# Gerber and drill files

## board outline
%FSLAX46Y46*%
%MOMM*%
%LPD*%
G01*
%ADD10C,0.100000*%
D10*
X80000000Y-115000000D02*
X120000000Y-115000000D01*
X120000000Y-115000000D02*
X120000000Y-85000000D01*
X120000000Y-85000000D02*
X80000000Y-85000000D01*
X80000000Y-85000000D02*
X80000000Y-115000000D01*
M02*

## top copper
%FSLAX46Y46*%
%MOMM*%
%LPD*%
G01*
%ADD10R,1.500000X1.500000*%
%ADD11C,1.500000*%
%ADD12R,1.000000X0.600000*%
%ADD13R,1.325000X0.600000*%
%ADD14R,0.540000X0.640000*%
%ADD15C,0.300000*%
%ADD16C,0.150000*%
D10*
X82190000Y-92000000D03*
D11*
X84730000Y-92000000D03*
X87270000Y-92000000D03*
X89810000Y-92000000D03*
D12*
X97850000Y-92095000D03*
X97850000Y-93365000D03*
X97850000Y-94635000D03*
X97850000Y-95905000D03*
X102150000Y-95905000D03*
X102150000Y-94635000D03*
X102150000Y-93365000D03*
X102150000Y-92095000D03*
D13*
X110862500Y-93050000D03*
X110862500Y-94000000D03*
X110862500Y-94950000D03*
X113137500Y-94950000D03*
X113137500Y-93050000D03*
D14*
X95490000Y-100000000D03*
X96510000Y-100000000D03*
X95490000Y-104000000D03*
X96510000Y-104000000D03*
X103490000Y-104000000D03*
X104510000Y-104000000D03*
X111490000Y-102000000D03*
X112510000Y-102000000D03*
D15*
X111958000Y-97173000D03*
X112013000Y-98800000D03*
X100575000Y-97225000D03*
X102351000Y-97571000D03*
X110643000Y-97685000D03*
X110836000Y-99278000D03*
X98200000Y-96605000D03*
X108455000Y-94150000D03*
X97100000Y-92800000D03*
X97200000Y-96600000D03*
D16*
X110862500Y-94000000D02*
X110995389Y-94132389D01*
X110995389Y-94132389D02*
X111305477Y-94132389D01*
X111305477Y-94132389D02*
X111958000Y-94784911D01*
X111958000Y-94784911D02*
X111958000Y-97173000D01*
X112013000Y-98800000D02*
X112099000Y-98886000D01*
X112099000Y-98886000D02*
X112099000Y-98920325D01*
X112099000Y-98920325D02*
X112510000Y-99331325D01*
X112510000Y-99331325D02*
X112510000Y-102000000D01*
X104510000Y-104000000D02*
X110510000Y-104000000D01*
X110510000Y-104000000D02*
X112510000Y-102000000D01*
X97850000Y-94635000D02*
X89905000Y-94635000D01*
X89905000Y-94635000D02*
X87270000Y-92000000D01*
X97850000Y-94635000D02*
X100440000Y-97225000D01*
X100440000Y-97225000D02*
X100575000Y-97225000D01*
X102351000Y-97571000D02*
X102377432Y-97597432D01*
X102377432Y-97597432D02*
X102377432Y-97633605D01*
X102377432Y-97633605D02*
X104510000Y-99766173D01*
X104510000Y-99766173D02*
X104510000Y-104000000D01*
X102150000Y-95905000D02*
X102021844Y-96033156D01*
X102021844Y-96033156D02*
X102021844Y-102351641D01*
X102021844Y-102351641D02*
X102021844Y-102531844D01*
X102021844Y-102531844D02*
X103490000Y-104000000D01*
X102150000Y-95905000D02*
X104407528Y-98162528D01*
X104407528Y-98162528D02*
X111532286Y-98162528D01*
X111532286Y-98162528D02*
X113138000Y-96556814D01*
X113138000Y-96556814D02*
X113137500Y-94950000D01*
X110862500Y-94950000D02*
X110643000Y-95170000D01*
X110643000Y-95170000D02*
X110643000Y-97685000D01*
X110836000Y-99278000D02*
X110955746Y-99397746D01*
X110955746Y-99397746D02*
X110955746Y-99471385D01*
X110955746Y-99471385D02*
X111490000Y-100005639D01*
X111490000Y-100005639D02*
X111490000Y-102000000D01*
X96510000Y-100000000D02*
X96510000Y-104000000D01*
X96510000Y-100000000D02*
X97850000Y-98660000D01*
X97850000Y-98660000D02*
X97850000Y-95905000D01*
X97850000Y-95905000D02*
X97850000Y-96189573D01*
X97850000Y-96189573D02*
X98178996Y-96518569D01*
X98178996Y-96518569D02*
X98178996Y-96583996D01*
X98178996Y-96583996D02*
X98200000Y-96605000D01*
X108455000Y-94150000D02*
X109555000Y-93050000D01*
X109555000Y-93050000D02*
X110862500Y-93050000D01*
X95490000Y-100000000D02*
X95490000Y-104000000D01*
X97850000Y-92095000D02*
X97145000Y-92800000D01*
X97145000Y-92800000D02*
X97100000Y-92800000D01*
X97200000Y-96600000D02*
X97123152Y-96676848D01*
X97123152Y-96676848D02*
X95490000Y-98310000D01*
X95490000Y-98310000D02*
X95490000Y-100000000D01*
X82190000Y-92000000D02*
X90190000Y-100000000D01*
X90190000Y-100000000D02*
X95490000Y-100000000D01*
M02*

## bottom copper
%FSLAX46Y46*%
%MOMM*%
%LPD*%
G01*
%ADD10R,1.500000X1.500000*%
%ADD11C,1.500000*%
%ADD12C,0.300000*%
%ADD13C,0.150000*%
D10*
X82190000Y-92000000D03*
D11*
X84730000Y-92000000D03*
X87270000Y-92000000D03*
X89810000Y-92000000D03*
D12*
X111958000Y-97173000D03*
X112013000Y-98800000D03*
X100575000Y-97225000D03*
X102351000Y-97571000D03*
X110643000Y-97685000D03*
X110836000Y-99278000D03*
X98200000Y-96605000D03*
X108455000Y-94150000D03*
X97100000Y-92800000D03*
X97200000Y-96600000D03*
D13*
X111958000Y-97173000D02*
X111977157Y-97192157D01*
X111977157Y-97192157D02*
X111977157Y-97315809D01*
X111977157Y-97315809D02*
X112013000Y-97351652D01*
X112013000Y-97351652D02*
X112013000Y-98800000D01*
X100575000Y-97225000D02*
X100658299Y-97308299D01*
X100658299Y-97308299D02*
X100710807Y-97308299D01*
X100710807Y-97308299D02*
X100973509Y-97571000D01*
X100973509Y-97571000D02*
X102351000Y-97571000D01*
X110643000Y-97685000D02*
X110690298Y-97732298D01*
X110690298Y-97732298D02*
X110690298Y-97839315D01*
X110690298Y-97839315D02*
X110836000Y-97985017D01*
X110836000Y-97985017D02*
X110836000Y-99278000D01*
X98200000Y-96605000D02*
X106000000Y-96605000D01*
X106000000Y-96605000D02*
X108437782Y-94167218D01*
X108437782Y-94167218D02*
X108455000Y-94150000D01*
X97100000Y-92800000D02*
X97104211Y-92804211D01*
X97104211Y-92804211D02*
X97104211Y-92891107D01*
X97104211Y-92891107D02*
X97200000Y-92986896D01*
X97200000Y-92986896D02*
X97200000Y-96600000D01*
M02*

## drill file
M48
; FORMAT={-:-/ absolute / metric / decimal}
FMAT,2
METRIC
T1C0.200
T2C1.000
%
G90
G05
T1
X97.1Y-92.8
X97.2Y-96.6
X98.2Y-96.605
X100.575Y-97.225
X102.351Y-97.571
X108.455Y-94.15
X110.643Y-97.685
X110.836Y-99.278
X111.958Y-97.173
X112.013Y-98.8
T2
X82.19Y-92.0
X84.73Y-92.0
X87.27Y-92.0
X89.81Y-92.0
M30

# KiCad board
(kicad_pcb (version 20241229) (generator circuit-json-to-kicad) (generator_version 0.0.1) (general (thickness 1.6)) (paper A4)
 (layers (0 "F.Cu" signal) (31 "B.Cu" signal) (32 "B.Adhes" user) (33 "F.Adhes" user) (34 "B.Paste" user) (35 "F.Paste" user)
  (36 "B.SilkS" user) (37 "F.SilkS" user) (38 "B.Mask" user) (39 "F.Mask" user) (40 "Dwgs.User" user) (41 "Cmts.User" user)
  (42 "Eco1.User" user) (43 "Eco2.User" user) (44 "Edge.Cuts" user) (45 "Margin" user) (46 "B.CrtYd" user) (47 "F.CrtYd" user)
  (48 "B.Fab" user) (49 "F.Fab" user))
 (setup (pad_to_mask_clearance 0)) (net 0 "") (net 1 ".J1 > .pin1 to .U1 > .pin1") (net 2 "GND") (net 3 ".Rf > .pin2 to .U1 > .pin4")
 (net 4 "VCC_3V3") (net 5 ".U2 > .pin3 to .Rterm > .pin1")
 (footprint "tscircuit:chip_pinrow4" (layer F.Cu) (at 86 92 0)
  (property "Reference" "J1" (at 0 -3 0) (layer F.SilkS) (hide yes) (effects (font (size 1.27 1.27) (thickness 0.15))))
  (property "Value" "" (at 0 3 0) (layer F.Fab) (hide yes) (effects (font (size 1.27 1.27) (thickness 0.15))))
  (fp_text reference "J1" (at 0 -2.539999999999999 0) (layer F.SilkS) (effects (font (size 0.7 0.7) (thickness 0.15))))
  (pad "1" thru_hole rect (at -3.8099999999999987 0 0) (size 1.5 1.5) (drill 1) (layers *.Cu *.Mask) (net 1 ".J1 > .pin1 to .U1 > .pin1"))
  (pad "2" thru_hole circle (at -1.2699999999999996 0 0) (size 1.5 1.5) (drill 1) (layers *.Cu *.Mask))
  (pad "3" thru_hole circle (at 1.2699999999999996 0 0) (size 1.5 1.5) (drill 1) (layers *.Cu *.Mask) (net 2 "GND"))
  (pad "4" thru_hole circle (at 3.8100000000000005 0 0) (size 1.5 1.5) (drill 1) (layers *.Cu *.Mask)))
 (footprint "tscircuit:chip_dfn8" (layer F.Cu) (at 100 94 0)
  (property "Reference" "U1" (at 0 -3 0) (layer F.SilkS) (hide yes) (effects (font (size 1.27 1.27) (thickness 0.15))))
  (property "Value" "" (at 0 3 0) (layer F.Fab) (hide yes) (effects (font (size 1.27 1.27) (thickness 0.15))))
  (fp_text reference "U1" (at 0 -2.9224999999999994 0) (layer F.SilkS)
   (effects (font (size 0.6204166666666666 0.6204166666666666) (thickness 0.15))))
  (pad "1" smd rect (at -2.15 -1.9050000000000002 0) (size 1 0.6) (layers F.Cu F.Paste F.Mask) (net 1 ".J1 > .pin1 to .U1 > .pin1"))
  (pad "2" smd rect (at -2.15 -0.6349999999999998 0) (size 1 0.6) (layers F.Cu F.Paste F.Mask))
  (pad "3" smd rect (at -2.15 0.6349999999999998 0) (size 1 0.6) (layers F.Cu F.Paste F.Mask) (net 2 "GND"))
  (pad "4" smd rect (at -2.15 1.9050000000000002 0) (size 1 0.6) (layers F.Cu F.Paste F.Mask) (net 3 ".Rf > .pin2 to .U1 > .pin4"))
  (pad "5" smd rect (at 2.15 1.9050000000000002 0) (size 1 0.6) (layers F.Cu F.Paste F.Mask) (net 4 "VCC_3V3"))
  (pad "6" smd rect (at 2.15 0.6349999999999998 0) (size 1 0.6) (layers F.Cu F.Paste F.Mask))
  (pad "7" smd rect (at 2.15 -0.6349999999999998 0) (size 1 0.6) (layers F.Cu F.Paste F.Mask))
  (pad "8" smd rect (at 2.15 -1.9050000000000002 0) (size 1 0.6) (layers F.Cu F.Paste F.Mask)))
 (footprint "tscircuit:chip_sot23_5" (layer F.Cu) (at 112 94 0)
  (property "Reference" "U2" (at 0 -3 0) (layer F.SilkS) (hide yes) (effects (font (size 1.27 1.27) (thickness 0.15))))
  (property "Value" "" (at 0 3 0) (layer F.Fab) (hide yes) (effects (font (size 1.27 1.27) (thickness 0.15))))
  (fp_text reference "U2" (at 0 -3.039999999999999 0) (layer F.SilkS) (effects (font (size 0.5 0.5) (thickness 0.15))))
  (pad "1" smd rect (at -1.1374999999999993 -0.9500000000000002 0) (size 1.325 0.6) (layers F.Cu F.Paste F.Mask)
   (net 3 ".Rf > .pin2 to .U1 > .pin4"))
  (pad "2" smd rect (at -1.1374999999999993 0 0) (size 1.325 0.6) (layers F.Cu F.Paste F.Mask) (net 2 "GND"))
  (pad "3" smd rect (at -1.1374999999999993 0.9500000000000002 0) (size 1.325 0.6) (layers F.Cu F.Paste F.Mask)
   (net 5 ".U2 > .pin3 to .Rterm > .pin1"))
  (pad "4" smd rect (at 1.1374999999999993 0.9500000000000002 0) (size 1.325 0.6) (layers F.Cu F.Paste F.Mask) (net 4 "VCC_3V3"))
  (pad "5" smd rect (at 1.1374999999999993 -0.9500000000000002 0) (size 1.325 0.6) (layers F.Cu F.Paste F.Mask)))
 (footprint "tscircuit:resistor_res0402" (layer F.Cu) (at 96 100 0)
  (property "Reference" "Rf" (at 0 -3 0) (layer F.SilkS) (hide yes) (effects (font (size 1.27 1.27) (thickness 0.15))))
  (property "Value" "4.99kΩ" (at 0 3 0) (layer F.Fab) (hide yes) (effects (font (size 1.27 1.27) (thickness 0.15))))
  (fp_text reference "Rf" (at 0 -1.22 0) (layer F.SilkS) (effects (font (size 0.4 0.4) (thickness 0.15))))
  (pad "1" smd rect (at -0.5099999999999998 0 0) (size 0.54 0.64) (layers F.Cu F.Paste F.Mask) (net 1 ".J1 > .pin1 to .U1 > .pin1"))
  (pad "2" smd rect (at 0.5099999999999998 0 0) (size 0.54 0.64) (layers F.Cu F.Paste F.Mask) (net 3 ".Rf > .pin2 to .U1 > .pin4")))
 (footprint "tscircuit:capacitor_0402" (layer F.Cu) (at 96 104 0)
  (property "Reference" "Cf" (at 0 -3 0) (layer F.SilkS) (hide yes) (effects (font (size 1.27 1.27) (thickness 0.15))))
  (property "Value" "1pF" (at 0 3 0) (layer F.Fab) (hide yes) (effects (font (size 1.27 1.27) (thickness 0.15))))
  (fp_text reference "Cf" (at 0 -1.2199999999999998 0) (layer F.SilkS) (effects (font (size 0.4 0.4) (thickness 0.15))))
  (pad "1" smd rect (at -0.5099999999999998 0 0) (size 0.54 0.64) (layers F.Cu F.Paste F.Mask) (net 1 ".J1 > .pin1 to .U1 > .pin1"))
  (pad "2" smd rect (at 0.5099999999999998 0 0) (size 0.54 0.64) (layers F.Cu F.Paste F.Mask) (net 3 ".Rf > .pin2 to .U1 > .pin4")))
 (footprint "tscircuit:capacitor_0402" (layer F.Cu) (at 104 104 0)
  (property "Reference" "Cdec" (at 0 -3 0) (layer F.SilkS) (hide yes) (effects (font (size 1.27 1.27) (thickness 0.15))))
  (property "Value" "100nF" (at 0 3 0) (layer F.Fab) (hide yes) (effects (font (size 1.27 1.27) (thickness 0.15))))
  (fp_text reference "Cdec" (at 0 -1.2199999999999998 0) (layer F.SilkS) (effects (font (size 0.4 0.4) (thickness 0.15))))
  (pad "1" smd rect (at -0.5099999999999998 0 0) (size 0.54 0.64) (layers F.Cu F.Paste F.Mask) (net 4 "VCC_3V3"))
  (pad "2" smd rect (at 0.5099999999999998 0 0) (size 0.54 0.64) (layers F.Cu F.Paste F.Mask) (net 2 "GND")))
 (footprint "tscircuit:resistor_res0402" (layer F.Cu) (at 112 102 0)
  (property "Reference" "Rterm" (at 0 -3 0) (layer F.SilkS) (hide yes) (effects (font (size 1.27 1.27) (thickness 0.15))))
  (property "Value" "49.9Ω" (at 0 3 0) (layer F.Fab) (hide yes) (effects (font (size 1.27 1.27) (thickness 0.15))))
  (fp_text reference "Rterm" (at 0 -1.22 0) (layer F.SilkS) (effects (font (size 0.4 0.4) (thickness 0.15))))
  (pad "1" smd rect (at -0.5099999999999998 0 0) (size 0.54 0.64) (layers F.Cu F.Paste F.Mask) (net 5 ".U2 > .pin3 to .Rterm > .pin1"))
  (pad "2" smd rect (at 0.5099999999999998 0 0) (size 0.54 0.64) (layers F.Cu F.Paste F.Mask) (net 2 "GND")))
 (segment (start 110.8625 94) (end 110.99538864191226 94.13238864191226) (width 0.15) (layer F.Cu) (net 2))
 (segment (start 110.99538864191226 94.13238864191226) (end 111.30547729531605 94.13238864191226) (width 0.15) (layer F.Cu) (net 2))
 (segment (start 111.30547729531605 94.13238864191226) (end 111.958 94.7849113465962) (width 0.15) (layer F.Cu) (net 2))
 (segment (start 111.958 94.7849113465962) (end 111.958 97.173) (width 0.15) (layer F.Cu) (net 2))
 (segment (start 111.958 97.173) (end 111.97715696330971 97.19215696330971) (width 0.15) (layer B.Cu) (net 2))
 (segment (start 111.97715696330971 97.19215696330971) (end 111.97715696330971 97.3158089003817) (width 0.15) (layer B.Cu) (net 2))
 (segment (start 111.97715696330971 97.3158089003817) (end 112.013 97.35165193707198) (width 0.15) (layer B.Cu) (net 2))
 (segment (start 112.013 97.35165193707198) (end 112.013 98.8) (width 0.15) (layer B.Cu) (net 2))
 (segment (start 112.013 98.8) (end 112.09899963028704 98.88599963028705) (width 0.15) (layer F.Cu) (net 2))
 (segment (start 112.09899963028704 98.88599963028705) (end 112.09899963028704 98.92032463784359) (width 0.15) (layer F.Cu) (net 2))
 (segment (start 112.09899963028704 98.92032463784359) (end 112.51 99.33132500755654) (width 0.15) (layer F.Cu) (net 2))
 (segment (start 112.51 99.33132500755654) (end 112.51 102) (width 0.15) (layer F.Cu) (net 2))
 (segment (start 104.51 104) (end 110.51 104) (width 0.15) (layer F.Cu) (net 2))
 (segment (start 110.51 104) (end 112.51 102) (width 0.15) (layer F.Cu) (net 2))
 (segment (start 97.85 94.635) (end 89.905 94.635) (width 0.15) (layer F.Cu) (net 2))
 (segment (start 89.905 94.635) (end 87.27 92) (width 0.15) (layer F.Cu) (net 2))
 (segment (start 97.85 94.635) (end 100.44 97.225) (width 0.15) (layer F.Cu) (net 2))
 (segment (start 100.44 97.225) (end 100.575 97.225) (width 0.15) (layer F.Cu) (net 2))
 (segment (start 100.575 97.225) (end 100.65829862620022 97.30829862620021) (width 0.15) (layer B.Cu) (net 2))
 (segment (start 100.65829862620022 97.30829862620021) (end 100.71080742886063 97.30829862620021) (width 0.15) (layer B.Cu) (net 2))
 (segment (start 100.71080742886063 97.30829862620021) (end 100.97350880266042 97.571) (width 0.15) (layer B.Cu) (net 2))
 (segment (start 100.97350880266042 97.571) (end 102.351 97.571) (width 0.15) (layer B.Cu) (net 2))
 (segment (start 102.351 97.571) (end 102.37743222737569 97.59743222737569) (width 0.15) (layer F.Cu) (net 2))
 (segment (start 102.37743222737569 97.59743222737569) (end 102.37743222737569 97.63360525070775) (width 0.15) (layer F.Cu) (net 2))
 (segment (start 102.37743222737569 97.63360525070775) (end 104.51 99.76617302333206) (width 0.15) (layer F.Cu) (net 2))
 (segment (start 104.51 99.76617302333206) (end 104.51 104) (width 0.15) (layer F.Cu) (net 2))
 (segment (start 102.15 95.905) (end 102.0218438922022 96.0331561077978) (width 0.15) (layer F.Cu) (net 4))
 (segment (start 102.0218438922022 96.0331561077978) (end 102.0218438922022 102.35164117935577) (width 0.15) (layer F.Cu) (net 4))
 (segment (start 102.0218438922022 102.35164117935577) (end 102.0218438922022 102.5318438922022) (width 0.15) (layer F.Cu) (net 4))
 (segment (start 102.0218438922022 102.5318438922022) (end 103.49 104) (width 0.15) (layer F.Cu) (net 4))
 (segment (start 102.15 95.905) (end 104.40752755203931 98.16252755203931) (width 0.15) (layer F.Cu) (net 4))
 (segment (start 104.40752755203931 98.16252755203931) (end 111.53228648019808 98.16252755203931) (width 0.15) (layer F.Cu) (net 4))
 (segment (start 111.53228648019808 98.16252755203931) (end 113.138 96.5568140322374) (width 0.15) (layer F.Cu) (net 4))
 (segment (start 113.138 96.5568140322374) (end 113.1375 94.95) (width 0.15) (layer F.Cu) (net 4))
 (segment (start 110.8625 94.95) (end 110.643 95.17) (width 0.15) (layer F.Cu) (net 5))
 (segment (start 110.643 95.17) (end 110.643 97.685) (width 0.15) (layer F.Cu) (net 5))
 (segment (start 110.643 97.685) (end 110.69029788521874 97.73229788521874) (width 0.15) (layer B.Cu) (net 5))
 (segment (start 110.69029788521874 97.73229788521874) (end 110.69029788521874 97.83931526836895) (width 0.15) (layer B.Cu) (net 5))
 (segment (start 110.69029788521874 97.83931526836895) (end 110.836 97.98501738315021) (width 0.15) (layer B.Cu) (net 5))
 (segment (start 110.836 97.98501738315021) (end 110.836 99.278) (width 0.15) (layer B.Cu) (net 5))
 (segment (start 110.836 99.278) (end 110.95574634516363 99.39774634516364) (width 0.15) (layer F.Cu) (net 5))
 (segment (start 110.95574634516363 99.39774634516364) (end 110.95574634516363 99.47138530493655) (width 0.15) (layer F.Cu) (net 5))
 (segment (start 110.95574634516363 99.47138530493655) (end 111.49 100.00563895977291) (width 0.15) (layer F.Cu) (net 5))
 (segment (start 111.49 100.00563895977291) (end 111.49 102) (width 0.15) (layer F.Cu) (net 5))
 (segment (start 96.51 100) (end 96.51 104) (width 0.15) (layer F.Cu) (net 3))
 (segment (start 96.51 100) (end 97.85 98.66) (width 0.15) (layer F.Cu) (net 3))
 (segment (start 97.85 98.66) (end 97.85 95.905) (width 0.15) (layer F.Cu) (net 3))
 (segment (start 97.85 95.905) (end 97.85 96.18957290456092) (width 0.15) (layer F.Cu) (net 3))
 (segment (start 97.85 96.18957290456092) (end 98.17899618381983 96.51856908838074) (width 0.15) (layer F.Cu) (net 3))
 (segment (start 98.17899618381983 96.51856908838074) (end 98.17899618381983 96.58399618381983) (width 0.15) (layer F.Cu) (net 3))
 (segment (start 98.17899618381983 96.58399618381983) (end 98.2 96.605) (width 0.15) (layer F.Cu) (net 3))
 (segment (start 98.2 96.605) (end 106 96.605) (width 0.15) (layer B.Cu) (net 3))
 (segment (start 106 96.605) (end 108.4377819599855 94.1672180400145) (width 0.15) (layer B.Cu) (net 3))
 (segment (start 108.4377819599855 94.1672180400145) (end 108.455 94.15) (width 0.15) (layer B.Cu) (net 3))
 (segment (start 108.455 94.15) (end 109.555 93.05) (width 0.15) (layer F.Cu) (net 3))
 (segment (start 109.555 93.05) (end 110.8625 93.05) (width 0.15) (layer F.Cu) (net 3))
 (segment (start 95.49 100) (end 95.49 104) (width 0.15) (layer F.Cu) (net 1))
 (segment (start 97.85 92.095) (end 97.145 92.8) (width 0.15) (layer F.Cu) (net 1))
 (segment (start 97.145 92.8) (end 97.1 92.8) (width 0.15) (layer F.Cu) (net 1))
 (segment (start 97.1 92.8) (end 97.10421113345926 92.80421113345925) (width 0.15) (layer B.Cu) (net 1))
 (segment (start 97.10421113345926 92.80421113345925) (end 97.10421113345926 92.89110668092891) (width 0.15) (layer B.Cu) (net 1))
 (segment (start 97.10421113345926 92.89110668092891) (end 97.2 92.98689554746966) (width 0.15) (layer B.Cu) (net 1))
 (segment (start 97.2 92.98689554746966) (end 97.2 96.6) (width 0.15) (layer B.Cu) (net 1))
 (segment (start 97.2 96.6) (end 97.12315195195319 96.6768480480468) (width 0.15) (layer F.Cu) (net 1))
 (segment (start 97.12315195195319 96.6768480480468) (end 95.49 98.31) (width 0.15) (layer F.Cu) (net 1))
 (segment (start 95.49 98.31) (end 95.49 100) (width 0.15) (layer F.Cu) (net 1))
 (segment (start 82.19 92) (end 90.19 100) (width 0.15) (layer F.Cu) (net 1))
 (segment (start 90.19 100) (end 95.49 100) (width 0.15) (layer F.Cu) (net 1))
 (gr_line (start 80 115) (end 120 115) (width 0.1) (layer Edge.Cuts))
 (gr_line (start 120 115) (end 120 85) (width 0.1) (layer Edge.Cuts))
 (gr_line (start 120 85) (end 80 85) (width 0.1) (layer Edge.Cuts))
 (gr_line (start 80 85) (end 80 115) (width 0.1) (layer Edge.Cuts))
 (via (at 111.958 97.173) (size 0.3) (drill 0.2) (layers F.Cu B.Cu) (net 2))
 (via (at 112.013 98.8) (size 0.3) (drill 0.2) (layers F.Cu B.Cu) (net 2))
 (via (at 100.575 97.225) (size 0.3) (drill 0.2) (layers F.Cu B.Cu) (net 2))
 (via (at 102.351 97.571) (size 0.3) (drill 0.2) (layers F.Cu B.Cu) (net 2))
 (via (at 110.643 97.685) (size 0.3) (drill 0.2) (layers F.Cu B.Cu) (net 5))
 (via (at 110.836 99.278) (size 0.3) (drill 0.2) (layers F.Cu B.Cu) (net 5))
 (via (at 98.2 96.605) (size 0.3) (drill 0.2) (layers F.Cu B.Cu) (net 3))
 (via (at 108.455 94.15) (size 0.3) (drill 0.2) (layers F.Cu B.Cu) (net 3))
 (via (at 97.1 92.8) (size 0.3) (drill 0.2) (layers F.Cu B.Cu) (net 1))
 (via (at 97.2 96.6) (size 0.3) (drill 0.2) (layers F.Cu B.Cu) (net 1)))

